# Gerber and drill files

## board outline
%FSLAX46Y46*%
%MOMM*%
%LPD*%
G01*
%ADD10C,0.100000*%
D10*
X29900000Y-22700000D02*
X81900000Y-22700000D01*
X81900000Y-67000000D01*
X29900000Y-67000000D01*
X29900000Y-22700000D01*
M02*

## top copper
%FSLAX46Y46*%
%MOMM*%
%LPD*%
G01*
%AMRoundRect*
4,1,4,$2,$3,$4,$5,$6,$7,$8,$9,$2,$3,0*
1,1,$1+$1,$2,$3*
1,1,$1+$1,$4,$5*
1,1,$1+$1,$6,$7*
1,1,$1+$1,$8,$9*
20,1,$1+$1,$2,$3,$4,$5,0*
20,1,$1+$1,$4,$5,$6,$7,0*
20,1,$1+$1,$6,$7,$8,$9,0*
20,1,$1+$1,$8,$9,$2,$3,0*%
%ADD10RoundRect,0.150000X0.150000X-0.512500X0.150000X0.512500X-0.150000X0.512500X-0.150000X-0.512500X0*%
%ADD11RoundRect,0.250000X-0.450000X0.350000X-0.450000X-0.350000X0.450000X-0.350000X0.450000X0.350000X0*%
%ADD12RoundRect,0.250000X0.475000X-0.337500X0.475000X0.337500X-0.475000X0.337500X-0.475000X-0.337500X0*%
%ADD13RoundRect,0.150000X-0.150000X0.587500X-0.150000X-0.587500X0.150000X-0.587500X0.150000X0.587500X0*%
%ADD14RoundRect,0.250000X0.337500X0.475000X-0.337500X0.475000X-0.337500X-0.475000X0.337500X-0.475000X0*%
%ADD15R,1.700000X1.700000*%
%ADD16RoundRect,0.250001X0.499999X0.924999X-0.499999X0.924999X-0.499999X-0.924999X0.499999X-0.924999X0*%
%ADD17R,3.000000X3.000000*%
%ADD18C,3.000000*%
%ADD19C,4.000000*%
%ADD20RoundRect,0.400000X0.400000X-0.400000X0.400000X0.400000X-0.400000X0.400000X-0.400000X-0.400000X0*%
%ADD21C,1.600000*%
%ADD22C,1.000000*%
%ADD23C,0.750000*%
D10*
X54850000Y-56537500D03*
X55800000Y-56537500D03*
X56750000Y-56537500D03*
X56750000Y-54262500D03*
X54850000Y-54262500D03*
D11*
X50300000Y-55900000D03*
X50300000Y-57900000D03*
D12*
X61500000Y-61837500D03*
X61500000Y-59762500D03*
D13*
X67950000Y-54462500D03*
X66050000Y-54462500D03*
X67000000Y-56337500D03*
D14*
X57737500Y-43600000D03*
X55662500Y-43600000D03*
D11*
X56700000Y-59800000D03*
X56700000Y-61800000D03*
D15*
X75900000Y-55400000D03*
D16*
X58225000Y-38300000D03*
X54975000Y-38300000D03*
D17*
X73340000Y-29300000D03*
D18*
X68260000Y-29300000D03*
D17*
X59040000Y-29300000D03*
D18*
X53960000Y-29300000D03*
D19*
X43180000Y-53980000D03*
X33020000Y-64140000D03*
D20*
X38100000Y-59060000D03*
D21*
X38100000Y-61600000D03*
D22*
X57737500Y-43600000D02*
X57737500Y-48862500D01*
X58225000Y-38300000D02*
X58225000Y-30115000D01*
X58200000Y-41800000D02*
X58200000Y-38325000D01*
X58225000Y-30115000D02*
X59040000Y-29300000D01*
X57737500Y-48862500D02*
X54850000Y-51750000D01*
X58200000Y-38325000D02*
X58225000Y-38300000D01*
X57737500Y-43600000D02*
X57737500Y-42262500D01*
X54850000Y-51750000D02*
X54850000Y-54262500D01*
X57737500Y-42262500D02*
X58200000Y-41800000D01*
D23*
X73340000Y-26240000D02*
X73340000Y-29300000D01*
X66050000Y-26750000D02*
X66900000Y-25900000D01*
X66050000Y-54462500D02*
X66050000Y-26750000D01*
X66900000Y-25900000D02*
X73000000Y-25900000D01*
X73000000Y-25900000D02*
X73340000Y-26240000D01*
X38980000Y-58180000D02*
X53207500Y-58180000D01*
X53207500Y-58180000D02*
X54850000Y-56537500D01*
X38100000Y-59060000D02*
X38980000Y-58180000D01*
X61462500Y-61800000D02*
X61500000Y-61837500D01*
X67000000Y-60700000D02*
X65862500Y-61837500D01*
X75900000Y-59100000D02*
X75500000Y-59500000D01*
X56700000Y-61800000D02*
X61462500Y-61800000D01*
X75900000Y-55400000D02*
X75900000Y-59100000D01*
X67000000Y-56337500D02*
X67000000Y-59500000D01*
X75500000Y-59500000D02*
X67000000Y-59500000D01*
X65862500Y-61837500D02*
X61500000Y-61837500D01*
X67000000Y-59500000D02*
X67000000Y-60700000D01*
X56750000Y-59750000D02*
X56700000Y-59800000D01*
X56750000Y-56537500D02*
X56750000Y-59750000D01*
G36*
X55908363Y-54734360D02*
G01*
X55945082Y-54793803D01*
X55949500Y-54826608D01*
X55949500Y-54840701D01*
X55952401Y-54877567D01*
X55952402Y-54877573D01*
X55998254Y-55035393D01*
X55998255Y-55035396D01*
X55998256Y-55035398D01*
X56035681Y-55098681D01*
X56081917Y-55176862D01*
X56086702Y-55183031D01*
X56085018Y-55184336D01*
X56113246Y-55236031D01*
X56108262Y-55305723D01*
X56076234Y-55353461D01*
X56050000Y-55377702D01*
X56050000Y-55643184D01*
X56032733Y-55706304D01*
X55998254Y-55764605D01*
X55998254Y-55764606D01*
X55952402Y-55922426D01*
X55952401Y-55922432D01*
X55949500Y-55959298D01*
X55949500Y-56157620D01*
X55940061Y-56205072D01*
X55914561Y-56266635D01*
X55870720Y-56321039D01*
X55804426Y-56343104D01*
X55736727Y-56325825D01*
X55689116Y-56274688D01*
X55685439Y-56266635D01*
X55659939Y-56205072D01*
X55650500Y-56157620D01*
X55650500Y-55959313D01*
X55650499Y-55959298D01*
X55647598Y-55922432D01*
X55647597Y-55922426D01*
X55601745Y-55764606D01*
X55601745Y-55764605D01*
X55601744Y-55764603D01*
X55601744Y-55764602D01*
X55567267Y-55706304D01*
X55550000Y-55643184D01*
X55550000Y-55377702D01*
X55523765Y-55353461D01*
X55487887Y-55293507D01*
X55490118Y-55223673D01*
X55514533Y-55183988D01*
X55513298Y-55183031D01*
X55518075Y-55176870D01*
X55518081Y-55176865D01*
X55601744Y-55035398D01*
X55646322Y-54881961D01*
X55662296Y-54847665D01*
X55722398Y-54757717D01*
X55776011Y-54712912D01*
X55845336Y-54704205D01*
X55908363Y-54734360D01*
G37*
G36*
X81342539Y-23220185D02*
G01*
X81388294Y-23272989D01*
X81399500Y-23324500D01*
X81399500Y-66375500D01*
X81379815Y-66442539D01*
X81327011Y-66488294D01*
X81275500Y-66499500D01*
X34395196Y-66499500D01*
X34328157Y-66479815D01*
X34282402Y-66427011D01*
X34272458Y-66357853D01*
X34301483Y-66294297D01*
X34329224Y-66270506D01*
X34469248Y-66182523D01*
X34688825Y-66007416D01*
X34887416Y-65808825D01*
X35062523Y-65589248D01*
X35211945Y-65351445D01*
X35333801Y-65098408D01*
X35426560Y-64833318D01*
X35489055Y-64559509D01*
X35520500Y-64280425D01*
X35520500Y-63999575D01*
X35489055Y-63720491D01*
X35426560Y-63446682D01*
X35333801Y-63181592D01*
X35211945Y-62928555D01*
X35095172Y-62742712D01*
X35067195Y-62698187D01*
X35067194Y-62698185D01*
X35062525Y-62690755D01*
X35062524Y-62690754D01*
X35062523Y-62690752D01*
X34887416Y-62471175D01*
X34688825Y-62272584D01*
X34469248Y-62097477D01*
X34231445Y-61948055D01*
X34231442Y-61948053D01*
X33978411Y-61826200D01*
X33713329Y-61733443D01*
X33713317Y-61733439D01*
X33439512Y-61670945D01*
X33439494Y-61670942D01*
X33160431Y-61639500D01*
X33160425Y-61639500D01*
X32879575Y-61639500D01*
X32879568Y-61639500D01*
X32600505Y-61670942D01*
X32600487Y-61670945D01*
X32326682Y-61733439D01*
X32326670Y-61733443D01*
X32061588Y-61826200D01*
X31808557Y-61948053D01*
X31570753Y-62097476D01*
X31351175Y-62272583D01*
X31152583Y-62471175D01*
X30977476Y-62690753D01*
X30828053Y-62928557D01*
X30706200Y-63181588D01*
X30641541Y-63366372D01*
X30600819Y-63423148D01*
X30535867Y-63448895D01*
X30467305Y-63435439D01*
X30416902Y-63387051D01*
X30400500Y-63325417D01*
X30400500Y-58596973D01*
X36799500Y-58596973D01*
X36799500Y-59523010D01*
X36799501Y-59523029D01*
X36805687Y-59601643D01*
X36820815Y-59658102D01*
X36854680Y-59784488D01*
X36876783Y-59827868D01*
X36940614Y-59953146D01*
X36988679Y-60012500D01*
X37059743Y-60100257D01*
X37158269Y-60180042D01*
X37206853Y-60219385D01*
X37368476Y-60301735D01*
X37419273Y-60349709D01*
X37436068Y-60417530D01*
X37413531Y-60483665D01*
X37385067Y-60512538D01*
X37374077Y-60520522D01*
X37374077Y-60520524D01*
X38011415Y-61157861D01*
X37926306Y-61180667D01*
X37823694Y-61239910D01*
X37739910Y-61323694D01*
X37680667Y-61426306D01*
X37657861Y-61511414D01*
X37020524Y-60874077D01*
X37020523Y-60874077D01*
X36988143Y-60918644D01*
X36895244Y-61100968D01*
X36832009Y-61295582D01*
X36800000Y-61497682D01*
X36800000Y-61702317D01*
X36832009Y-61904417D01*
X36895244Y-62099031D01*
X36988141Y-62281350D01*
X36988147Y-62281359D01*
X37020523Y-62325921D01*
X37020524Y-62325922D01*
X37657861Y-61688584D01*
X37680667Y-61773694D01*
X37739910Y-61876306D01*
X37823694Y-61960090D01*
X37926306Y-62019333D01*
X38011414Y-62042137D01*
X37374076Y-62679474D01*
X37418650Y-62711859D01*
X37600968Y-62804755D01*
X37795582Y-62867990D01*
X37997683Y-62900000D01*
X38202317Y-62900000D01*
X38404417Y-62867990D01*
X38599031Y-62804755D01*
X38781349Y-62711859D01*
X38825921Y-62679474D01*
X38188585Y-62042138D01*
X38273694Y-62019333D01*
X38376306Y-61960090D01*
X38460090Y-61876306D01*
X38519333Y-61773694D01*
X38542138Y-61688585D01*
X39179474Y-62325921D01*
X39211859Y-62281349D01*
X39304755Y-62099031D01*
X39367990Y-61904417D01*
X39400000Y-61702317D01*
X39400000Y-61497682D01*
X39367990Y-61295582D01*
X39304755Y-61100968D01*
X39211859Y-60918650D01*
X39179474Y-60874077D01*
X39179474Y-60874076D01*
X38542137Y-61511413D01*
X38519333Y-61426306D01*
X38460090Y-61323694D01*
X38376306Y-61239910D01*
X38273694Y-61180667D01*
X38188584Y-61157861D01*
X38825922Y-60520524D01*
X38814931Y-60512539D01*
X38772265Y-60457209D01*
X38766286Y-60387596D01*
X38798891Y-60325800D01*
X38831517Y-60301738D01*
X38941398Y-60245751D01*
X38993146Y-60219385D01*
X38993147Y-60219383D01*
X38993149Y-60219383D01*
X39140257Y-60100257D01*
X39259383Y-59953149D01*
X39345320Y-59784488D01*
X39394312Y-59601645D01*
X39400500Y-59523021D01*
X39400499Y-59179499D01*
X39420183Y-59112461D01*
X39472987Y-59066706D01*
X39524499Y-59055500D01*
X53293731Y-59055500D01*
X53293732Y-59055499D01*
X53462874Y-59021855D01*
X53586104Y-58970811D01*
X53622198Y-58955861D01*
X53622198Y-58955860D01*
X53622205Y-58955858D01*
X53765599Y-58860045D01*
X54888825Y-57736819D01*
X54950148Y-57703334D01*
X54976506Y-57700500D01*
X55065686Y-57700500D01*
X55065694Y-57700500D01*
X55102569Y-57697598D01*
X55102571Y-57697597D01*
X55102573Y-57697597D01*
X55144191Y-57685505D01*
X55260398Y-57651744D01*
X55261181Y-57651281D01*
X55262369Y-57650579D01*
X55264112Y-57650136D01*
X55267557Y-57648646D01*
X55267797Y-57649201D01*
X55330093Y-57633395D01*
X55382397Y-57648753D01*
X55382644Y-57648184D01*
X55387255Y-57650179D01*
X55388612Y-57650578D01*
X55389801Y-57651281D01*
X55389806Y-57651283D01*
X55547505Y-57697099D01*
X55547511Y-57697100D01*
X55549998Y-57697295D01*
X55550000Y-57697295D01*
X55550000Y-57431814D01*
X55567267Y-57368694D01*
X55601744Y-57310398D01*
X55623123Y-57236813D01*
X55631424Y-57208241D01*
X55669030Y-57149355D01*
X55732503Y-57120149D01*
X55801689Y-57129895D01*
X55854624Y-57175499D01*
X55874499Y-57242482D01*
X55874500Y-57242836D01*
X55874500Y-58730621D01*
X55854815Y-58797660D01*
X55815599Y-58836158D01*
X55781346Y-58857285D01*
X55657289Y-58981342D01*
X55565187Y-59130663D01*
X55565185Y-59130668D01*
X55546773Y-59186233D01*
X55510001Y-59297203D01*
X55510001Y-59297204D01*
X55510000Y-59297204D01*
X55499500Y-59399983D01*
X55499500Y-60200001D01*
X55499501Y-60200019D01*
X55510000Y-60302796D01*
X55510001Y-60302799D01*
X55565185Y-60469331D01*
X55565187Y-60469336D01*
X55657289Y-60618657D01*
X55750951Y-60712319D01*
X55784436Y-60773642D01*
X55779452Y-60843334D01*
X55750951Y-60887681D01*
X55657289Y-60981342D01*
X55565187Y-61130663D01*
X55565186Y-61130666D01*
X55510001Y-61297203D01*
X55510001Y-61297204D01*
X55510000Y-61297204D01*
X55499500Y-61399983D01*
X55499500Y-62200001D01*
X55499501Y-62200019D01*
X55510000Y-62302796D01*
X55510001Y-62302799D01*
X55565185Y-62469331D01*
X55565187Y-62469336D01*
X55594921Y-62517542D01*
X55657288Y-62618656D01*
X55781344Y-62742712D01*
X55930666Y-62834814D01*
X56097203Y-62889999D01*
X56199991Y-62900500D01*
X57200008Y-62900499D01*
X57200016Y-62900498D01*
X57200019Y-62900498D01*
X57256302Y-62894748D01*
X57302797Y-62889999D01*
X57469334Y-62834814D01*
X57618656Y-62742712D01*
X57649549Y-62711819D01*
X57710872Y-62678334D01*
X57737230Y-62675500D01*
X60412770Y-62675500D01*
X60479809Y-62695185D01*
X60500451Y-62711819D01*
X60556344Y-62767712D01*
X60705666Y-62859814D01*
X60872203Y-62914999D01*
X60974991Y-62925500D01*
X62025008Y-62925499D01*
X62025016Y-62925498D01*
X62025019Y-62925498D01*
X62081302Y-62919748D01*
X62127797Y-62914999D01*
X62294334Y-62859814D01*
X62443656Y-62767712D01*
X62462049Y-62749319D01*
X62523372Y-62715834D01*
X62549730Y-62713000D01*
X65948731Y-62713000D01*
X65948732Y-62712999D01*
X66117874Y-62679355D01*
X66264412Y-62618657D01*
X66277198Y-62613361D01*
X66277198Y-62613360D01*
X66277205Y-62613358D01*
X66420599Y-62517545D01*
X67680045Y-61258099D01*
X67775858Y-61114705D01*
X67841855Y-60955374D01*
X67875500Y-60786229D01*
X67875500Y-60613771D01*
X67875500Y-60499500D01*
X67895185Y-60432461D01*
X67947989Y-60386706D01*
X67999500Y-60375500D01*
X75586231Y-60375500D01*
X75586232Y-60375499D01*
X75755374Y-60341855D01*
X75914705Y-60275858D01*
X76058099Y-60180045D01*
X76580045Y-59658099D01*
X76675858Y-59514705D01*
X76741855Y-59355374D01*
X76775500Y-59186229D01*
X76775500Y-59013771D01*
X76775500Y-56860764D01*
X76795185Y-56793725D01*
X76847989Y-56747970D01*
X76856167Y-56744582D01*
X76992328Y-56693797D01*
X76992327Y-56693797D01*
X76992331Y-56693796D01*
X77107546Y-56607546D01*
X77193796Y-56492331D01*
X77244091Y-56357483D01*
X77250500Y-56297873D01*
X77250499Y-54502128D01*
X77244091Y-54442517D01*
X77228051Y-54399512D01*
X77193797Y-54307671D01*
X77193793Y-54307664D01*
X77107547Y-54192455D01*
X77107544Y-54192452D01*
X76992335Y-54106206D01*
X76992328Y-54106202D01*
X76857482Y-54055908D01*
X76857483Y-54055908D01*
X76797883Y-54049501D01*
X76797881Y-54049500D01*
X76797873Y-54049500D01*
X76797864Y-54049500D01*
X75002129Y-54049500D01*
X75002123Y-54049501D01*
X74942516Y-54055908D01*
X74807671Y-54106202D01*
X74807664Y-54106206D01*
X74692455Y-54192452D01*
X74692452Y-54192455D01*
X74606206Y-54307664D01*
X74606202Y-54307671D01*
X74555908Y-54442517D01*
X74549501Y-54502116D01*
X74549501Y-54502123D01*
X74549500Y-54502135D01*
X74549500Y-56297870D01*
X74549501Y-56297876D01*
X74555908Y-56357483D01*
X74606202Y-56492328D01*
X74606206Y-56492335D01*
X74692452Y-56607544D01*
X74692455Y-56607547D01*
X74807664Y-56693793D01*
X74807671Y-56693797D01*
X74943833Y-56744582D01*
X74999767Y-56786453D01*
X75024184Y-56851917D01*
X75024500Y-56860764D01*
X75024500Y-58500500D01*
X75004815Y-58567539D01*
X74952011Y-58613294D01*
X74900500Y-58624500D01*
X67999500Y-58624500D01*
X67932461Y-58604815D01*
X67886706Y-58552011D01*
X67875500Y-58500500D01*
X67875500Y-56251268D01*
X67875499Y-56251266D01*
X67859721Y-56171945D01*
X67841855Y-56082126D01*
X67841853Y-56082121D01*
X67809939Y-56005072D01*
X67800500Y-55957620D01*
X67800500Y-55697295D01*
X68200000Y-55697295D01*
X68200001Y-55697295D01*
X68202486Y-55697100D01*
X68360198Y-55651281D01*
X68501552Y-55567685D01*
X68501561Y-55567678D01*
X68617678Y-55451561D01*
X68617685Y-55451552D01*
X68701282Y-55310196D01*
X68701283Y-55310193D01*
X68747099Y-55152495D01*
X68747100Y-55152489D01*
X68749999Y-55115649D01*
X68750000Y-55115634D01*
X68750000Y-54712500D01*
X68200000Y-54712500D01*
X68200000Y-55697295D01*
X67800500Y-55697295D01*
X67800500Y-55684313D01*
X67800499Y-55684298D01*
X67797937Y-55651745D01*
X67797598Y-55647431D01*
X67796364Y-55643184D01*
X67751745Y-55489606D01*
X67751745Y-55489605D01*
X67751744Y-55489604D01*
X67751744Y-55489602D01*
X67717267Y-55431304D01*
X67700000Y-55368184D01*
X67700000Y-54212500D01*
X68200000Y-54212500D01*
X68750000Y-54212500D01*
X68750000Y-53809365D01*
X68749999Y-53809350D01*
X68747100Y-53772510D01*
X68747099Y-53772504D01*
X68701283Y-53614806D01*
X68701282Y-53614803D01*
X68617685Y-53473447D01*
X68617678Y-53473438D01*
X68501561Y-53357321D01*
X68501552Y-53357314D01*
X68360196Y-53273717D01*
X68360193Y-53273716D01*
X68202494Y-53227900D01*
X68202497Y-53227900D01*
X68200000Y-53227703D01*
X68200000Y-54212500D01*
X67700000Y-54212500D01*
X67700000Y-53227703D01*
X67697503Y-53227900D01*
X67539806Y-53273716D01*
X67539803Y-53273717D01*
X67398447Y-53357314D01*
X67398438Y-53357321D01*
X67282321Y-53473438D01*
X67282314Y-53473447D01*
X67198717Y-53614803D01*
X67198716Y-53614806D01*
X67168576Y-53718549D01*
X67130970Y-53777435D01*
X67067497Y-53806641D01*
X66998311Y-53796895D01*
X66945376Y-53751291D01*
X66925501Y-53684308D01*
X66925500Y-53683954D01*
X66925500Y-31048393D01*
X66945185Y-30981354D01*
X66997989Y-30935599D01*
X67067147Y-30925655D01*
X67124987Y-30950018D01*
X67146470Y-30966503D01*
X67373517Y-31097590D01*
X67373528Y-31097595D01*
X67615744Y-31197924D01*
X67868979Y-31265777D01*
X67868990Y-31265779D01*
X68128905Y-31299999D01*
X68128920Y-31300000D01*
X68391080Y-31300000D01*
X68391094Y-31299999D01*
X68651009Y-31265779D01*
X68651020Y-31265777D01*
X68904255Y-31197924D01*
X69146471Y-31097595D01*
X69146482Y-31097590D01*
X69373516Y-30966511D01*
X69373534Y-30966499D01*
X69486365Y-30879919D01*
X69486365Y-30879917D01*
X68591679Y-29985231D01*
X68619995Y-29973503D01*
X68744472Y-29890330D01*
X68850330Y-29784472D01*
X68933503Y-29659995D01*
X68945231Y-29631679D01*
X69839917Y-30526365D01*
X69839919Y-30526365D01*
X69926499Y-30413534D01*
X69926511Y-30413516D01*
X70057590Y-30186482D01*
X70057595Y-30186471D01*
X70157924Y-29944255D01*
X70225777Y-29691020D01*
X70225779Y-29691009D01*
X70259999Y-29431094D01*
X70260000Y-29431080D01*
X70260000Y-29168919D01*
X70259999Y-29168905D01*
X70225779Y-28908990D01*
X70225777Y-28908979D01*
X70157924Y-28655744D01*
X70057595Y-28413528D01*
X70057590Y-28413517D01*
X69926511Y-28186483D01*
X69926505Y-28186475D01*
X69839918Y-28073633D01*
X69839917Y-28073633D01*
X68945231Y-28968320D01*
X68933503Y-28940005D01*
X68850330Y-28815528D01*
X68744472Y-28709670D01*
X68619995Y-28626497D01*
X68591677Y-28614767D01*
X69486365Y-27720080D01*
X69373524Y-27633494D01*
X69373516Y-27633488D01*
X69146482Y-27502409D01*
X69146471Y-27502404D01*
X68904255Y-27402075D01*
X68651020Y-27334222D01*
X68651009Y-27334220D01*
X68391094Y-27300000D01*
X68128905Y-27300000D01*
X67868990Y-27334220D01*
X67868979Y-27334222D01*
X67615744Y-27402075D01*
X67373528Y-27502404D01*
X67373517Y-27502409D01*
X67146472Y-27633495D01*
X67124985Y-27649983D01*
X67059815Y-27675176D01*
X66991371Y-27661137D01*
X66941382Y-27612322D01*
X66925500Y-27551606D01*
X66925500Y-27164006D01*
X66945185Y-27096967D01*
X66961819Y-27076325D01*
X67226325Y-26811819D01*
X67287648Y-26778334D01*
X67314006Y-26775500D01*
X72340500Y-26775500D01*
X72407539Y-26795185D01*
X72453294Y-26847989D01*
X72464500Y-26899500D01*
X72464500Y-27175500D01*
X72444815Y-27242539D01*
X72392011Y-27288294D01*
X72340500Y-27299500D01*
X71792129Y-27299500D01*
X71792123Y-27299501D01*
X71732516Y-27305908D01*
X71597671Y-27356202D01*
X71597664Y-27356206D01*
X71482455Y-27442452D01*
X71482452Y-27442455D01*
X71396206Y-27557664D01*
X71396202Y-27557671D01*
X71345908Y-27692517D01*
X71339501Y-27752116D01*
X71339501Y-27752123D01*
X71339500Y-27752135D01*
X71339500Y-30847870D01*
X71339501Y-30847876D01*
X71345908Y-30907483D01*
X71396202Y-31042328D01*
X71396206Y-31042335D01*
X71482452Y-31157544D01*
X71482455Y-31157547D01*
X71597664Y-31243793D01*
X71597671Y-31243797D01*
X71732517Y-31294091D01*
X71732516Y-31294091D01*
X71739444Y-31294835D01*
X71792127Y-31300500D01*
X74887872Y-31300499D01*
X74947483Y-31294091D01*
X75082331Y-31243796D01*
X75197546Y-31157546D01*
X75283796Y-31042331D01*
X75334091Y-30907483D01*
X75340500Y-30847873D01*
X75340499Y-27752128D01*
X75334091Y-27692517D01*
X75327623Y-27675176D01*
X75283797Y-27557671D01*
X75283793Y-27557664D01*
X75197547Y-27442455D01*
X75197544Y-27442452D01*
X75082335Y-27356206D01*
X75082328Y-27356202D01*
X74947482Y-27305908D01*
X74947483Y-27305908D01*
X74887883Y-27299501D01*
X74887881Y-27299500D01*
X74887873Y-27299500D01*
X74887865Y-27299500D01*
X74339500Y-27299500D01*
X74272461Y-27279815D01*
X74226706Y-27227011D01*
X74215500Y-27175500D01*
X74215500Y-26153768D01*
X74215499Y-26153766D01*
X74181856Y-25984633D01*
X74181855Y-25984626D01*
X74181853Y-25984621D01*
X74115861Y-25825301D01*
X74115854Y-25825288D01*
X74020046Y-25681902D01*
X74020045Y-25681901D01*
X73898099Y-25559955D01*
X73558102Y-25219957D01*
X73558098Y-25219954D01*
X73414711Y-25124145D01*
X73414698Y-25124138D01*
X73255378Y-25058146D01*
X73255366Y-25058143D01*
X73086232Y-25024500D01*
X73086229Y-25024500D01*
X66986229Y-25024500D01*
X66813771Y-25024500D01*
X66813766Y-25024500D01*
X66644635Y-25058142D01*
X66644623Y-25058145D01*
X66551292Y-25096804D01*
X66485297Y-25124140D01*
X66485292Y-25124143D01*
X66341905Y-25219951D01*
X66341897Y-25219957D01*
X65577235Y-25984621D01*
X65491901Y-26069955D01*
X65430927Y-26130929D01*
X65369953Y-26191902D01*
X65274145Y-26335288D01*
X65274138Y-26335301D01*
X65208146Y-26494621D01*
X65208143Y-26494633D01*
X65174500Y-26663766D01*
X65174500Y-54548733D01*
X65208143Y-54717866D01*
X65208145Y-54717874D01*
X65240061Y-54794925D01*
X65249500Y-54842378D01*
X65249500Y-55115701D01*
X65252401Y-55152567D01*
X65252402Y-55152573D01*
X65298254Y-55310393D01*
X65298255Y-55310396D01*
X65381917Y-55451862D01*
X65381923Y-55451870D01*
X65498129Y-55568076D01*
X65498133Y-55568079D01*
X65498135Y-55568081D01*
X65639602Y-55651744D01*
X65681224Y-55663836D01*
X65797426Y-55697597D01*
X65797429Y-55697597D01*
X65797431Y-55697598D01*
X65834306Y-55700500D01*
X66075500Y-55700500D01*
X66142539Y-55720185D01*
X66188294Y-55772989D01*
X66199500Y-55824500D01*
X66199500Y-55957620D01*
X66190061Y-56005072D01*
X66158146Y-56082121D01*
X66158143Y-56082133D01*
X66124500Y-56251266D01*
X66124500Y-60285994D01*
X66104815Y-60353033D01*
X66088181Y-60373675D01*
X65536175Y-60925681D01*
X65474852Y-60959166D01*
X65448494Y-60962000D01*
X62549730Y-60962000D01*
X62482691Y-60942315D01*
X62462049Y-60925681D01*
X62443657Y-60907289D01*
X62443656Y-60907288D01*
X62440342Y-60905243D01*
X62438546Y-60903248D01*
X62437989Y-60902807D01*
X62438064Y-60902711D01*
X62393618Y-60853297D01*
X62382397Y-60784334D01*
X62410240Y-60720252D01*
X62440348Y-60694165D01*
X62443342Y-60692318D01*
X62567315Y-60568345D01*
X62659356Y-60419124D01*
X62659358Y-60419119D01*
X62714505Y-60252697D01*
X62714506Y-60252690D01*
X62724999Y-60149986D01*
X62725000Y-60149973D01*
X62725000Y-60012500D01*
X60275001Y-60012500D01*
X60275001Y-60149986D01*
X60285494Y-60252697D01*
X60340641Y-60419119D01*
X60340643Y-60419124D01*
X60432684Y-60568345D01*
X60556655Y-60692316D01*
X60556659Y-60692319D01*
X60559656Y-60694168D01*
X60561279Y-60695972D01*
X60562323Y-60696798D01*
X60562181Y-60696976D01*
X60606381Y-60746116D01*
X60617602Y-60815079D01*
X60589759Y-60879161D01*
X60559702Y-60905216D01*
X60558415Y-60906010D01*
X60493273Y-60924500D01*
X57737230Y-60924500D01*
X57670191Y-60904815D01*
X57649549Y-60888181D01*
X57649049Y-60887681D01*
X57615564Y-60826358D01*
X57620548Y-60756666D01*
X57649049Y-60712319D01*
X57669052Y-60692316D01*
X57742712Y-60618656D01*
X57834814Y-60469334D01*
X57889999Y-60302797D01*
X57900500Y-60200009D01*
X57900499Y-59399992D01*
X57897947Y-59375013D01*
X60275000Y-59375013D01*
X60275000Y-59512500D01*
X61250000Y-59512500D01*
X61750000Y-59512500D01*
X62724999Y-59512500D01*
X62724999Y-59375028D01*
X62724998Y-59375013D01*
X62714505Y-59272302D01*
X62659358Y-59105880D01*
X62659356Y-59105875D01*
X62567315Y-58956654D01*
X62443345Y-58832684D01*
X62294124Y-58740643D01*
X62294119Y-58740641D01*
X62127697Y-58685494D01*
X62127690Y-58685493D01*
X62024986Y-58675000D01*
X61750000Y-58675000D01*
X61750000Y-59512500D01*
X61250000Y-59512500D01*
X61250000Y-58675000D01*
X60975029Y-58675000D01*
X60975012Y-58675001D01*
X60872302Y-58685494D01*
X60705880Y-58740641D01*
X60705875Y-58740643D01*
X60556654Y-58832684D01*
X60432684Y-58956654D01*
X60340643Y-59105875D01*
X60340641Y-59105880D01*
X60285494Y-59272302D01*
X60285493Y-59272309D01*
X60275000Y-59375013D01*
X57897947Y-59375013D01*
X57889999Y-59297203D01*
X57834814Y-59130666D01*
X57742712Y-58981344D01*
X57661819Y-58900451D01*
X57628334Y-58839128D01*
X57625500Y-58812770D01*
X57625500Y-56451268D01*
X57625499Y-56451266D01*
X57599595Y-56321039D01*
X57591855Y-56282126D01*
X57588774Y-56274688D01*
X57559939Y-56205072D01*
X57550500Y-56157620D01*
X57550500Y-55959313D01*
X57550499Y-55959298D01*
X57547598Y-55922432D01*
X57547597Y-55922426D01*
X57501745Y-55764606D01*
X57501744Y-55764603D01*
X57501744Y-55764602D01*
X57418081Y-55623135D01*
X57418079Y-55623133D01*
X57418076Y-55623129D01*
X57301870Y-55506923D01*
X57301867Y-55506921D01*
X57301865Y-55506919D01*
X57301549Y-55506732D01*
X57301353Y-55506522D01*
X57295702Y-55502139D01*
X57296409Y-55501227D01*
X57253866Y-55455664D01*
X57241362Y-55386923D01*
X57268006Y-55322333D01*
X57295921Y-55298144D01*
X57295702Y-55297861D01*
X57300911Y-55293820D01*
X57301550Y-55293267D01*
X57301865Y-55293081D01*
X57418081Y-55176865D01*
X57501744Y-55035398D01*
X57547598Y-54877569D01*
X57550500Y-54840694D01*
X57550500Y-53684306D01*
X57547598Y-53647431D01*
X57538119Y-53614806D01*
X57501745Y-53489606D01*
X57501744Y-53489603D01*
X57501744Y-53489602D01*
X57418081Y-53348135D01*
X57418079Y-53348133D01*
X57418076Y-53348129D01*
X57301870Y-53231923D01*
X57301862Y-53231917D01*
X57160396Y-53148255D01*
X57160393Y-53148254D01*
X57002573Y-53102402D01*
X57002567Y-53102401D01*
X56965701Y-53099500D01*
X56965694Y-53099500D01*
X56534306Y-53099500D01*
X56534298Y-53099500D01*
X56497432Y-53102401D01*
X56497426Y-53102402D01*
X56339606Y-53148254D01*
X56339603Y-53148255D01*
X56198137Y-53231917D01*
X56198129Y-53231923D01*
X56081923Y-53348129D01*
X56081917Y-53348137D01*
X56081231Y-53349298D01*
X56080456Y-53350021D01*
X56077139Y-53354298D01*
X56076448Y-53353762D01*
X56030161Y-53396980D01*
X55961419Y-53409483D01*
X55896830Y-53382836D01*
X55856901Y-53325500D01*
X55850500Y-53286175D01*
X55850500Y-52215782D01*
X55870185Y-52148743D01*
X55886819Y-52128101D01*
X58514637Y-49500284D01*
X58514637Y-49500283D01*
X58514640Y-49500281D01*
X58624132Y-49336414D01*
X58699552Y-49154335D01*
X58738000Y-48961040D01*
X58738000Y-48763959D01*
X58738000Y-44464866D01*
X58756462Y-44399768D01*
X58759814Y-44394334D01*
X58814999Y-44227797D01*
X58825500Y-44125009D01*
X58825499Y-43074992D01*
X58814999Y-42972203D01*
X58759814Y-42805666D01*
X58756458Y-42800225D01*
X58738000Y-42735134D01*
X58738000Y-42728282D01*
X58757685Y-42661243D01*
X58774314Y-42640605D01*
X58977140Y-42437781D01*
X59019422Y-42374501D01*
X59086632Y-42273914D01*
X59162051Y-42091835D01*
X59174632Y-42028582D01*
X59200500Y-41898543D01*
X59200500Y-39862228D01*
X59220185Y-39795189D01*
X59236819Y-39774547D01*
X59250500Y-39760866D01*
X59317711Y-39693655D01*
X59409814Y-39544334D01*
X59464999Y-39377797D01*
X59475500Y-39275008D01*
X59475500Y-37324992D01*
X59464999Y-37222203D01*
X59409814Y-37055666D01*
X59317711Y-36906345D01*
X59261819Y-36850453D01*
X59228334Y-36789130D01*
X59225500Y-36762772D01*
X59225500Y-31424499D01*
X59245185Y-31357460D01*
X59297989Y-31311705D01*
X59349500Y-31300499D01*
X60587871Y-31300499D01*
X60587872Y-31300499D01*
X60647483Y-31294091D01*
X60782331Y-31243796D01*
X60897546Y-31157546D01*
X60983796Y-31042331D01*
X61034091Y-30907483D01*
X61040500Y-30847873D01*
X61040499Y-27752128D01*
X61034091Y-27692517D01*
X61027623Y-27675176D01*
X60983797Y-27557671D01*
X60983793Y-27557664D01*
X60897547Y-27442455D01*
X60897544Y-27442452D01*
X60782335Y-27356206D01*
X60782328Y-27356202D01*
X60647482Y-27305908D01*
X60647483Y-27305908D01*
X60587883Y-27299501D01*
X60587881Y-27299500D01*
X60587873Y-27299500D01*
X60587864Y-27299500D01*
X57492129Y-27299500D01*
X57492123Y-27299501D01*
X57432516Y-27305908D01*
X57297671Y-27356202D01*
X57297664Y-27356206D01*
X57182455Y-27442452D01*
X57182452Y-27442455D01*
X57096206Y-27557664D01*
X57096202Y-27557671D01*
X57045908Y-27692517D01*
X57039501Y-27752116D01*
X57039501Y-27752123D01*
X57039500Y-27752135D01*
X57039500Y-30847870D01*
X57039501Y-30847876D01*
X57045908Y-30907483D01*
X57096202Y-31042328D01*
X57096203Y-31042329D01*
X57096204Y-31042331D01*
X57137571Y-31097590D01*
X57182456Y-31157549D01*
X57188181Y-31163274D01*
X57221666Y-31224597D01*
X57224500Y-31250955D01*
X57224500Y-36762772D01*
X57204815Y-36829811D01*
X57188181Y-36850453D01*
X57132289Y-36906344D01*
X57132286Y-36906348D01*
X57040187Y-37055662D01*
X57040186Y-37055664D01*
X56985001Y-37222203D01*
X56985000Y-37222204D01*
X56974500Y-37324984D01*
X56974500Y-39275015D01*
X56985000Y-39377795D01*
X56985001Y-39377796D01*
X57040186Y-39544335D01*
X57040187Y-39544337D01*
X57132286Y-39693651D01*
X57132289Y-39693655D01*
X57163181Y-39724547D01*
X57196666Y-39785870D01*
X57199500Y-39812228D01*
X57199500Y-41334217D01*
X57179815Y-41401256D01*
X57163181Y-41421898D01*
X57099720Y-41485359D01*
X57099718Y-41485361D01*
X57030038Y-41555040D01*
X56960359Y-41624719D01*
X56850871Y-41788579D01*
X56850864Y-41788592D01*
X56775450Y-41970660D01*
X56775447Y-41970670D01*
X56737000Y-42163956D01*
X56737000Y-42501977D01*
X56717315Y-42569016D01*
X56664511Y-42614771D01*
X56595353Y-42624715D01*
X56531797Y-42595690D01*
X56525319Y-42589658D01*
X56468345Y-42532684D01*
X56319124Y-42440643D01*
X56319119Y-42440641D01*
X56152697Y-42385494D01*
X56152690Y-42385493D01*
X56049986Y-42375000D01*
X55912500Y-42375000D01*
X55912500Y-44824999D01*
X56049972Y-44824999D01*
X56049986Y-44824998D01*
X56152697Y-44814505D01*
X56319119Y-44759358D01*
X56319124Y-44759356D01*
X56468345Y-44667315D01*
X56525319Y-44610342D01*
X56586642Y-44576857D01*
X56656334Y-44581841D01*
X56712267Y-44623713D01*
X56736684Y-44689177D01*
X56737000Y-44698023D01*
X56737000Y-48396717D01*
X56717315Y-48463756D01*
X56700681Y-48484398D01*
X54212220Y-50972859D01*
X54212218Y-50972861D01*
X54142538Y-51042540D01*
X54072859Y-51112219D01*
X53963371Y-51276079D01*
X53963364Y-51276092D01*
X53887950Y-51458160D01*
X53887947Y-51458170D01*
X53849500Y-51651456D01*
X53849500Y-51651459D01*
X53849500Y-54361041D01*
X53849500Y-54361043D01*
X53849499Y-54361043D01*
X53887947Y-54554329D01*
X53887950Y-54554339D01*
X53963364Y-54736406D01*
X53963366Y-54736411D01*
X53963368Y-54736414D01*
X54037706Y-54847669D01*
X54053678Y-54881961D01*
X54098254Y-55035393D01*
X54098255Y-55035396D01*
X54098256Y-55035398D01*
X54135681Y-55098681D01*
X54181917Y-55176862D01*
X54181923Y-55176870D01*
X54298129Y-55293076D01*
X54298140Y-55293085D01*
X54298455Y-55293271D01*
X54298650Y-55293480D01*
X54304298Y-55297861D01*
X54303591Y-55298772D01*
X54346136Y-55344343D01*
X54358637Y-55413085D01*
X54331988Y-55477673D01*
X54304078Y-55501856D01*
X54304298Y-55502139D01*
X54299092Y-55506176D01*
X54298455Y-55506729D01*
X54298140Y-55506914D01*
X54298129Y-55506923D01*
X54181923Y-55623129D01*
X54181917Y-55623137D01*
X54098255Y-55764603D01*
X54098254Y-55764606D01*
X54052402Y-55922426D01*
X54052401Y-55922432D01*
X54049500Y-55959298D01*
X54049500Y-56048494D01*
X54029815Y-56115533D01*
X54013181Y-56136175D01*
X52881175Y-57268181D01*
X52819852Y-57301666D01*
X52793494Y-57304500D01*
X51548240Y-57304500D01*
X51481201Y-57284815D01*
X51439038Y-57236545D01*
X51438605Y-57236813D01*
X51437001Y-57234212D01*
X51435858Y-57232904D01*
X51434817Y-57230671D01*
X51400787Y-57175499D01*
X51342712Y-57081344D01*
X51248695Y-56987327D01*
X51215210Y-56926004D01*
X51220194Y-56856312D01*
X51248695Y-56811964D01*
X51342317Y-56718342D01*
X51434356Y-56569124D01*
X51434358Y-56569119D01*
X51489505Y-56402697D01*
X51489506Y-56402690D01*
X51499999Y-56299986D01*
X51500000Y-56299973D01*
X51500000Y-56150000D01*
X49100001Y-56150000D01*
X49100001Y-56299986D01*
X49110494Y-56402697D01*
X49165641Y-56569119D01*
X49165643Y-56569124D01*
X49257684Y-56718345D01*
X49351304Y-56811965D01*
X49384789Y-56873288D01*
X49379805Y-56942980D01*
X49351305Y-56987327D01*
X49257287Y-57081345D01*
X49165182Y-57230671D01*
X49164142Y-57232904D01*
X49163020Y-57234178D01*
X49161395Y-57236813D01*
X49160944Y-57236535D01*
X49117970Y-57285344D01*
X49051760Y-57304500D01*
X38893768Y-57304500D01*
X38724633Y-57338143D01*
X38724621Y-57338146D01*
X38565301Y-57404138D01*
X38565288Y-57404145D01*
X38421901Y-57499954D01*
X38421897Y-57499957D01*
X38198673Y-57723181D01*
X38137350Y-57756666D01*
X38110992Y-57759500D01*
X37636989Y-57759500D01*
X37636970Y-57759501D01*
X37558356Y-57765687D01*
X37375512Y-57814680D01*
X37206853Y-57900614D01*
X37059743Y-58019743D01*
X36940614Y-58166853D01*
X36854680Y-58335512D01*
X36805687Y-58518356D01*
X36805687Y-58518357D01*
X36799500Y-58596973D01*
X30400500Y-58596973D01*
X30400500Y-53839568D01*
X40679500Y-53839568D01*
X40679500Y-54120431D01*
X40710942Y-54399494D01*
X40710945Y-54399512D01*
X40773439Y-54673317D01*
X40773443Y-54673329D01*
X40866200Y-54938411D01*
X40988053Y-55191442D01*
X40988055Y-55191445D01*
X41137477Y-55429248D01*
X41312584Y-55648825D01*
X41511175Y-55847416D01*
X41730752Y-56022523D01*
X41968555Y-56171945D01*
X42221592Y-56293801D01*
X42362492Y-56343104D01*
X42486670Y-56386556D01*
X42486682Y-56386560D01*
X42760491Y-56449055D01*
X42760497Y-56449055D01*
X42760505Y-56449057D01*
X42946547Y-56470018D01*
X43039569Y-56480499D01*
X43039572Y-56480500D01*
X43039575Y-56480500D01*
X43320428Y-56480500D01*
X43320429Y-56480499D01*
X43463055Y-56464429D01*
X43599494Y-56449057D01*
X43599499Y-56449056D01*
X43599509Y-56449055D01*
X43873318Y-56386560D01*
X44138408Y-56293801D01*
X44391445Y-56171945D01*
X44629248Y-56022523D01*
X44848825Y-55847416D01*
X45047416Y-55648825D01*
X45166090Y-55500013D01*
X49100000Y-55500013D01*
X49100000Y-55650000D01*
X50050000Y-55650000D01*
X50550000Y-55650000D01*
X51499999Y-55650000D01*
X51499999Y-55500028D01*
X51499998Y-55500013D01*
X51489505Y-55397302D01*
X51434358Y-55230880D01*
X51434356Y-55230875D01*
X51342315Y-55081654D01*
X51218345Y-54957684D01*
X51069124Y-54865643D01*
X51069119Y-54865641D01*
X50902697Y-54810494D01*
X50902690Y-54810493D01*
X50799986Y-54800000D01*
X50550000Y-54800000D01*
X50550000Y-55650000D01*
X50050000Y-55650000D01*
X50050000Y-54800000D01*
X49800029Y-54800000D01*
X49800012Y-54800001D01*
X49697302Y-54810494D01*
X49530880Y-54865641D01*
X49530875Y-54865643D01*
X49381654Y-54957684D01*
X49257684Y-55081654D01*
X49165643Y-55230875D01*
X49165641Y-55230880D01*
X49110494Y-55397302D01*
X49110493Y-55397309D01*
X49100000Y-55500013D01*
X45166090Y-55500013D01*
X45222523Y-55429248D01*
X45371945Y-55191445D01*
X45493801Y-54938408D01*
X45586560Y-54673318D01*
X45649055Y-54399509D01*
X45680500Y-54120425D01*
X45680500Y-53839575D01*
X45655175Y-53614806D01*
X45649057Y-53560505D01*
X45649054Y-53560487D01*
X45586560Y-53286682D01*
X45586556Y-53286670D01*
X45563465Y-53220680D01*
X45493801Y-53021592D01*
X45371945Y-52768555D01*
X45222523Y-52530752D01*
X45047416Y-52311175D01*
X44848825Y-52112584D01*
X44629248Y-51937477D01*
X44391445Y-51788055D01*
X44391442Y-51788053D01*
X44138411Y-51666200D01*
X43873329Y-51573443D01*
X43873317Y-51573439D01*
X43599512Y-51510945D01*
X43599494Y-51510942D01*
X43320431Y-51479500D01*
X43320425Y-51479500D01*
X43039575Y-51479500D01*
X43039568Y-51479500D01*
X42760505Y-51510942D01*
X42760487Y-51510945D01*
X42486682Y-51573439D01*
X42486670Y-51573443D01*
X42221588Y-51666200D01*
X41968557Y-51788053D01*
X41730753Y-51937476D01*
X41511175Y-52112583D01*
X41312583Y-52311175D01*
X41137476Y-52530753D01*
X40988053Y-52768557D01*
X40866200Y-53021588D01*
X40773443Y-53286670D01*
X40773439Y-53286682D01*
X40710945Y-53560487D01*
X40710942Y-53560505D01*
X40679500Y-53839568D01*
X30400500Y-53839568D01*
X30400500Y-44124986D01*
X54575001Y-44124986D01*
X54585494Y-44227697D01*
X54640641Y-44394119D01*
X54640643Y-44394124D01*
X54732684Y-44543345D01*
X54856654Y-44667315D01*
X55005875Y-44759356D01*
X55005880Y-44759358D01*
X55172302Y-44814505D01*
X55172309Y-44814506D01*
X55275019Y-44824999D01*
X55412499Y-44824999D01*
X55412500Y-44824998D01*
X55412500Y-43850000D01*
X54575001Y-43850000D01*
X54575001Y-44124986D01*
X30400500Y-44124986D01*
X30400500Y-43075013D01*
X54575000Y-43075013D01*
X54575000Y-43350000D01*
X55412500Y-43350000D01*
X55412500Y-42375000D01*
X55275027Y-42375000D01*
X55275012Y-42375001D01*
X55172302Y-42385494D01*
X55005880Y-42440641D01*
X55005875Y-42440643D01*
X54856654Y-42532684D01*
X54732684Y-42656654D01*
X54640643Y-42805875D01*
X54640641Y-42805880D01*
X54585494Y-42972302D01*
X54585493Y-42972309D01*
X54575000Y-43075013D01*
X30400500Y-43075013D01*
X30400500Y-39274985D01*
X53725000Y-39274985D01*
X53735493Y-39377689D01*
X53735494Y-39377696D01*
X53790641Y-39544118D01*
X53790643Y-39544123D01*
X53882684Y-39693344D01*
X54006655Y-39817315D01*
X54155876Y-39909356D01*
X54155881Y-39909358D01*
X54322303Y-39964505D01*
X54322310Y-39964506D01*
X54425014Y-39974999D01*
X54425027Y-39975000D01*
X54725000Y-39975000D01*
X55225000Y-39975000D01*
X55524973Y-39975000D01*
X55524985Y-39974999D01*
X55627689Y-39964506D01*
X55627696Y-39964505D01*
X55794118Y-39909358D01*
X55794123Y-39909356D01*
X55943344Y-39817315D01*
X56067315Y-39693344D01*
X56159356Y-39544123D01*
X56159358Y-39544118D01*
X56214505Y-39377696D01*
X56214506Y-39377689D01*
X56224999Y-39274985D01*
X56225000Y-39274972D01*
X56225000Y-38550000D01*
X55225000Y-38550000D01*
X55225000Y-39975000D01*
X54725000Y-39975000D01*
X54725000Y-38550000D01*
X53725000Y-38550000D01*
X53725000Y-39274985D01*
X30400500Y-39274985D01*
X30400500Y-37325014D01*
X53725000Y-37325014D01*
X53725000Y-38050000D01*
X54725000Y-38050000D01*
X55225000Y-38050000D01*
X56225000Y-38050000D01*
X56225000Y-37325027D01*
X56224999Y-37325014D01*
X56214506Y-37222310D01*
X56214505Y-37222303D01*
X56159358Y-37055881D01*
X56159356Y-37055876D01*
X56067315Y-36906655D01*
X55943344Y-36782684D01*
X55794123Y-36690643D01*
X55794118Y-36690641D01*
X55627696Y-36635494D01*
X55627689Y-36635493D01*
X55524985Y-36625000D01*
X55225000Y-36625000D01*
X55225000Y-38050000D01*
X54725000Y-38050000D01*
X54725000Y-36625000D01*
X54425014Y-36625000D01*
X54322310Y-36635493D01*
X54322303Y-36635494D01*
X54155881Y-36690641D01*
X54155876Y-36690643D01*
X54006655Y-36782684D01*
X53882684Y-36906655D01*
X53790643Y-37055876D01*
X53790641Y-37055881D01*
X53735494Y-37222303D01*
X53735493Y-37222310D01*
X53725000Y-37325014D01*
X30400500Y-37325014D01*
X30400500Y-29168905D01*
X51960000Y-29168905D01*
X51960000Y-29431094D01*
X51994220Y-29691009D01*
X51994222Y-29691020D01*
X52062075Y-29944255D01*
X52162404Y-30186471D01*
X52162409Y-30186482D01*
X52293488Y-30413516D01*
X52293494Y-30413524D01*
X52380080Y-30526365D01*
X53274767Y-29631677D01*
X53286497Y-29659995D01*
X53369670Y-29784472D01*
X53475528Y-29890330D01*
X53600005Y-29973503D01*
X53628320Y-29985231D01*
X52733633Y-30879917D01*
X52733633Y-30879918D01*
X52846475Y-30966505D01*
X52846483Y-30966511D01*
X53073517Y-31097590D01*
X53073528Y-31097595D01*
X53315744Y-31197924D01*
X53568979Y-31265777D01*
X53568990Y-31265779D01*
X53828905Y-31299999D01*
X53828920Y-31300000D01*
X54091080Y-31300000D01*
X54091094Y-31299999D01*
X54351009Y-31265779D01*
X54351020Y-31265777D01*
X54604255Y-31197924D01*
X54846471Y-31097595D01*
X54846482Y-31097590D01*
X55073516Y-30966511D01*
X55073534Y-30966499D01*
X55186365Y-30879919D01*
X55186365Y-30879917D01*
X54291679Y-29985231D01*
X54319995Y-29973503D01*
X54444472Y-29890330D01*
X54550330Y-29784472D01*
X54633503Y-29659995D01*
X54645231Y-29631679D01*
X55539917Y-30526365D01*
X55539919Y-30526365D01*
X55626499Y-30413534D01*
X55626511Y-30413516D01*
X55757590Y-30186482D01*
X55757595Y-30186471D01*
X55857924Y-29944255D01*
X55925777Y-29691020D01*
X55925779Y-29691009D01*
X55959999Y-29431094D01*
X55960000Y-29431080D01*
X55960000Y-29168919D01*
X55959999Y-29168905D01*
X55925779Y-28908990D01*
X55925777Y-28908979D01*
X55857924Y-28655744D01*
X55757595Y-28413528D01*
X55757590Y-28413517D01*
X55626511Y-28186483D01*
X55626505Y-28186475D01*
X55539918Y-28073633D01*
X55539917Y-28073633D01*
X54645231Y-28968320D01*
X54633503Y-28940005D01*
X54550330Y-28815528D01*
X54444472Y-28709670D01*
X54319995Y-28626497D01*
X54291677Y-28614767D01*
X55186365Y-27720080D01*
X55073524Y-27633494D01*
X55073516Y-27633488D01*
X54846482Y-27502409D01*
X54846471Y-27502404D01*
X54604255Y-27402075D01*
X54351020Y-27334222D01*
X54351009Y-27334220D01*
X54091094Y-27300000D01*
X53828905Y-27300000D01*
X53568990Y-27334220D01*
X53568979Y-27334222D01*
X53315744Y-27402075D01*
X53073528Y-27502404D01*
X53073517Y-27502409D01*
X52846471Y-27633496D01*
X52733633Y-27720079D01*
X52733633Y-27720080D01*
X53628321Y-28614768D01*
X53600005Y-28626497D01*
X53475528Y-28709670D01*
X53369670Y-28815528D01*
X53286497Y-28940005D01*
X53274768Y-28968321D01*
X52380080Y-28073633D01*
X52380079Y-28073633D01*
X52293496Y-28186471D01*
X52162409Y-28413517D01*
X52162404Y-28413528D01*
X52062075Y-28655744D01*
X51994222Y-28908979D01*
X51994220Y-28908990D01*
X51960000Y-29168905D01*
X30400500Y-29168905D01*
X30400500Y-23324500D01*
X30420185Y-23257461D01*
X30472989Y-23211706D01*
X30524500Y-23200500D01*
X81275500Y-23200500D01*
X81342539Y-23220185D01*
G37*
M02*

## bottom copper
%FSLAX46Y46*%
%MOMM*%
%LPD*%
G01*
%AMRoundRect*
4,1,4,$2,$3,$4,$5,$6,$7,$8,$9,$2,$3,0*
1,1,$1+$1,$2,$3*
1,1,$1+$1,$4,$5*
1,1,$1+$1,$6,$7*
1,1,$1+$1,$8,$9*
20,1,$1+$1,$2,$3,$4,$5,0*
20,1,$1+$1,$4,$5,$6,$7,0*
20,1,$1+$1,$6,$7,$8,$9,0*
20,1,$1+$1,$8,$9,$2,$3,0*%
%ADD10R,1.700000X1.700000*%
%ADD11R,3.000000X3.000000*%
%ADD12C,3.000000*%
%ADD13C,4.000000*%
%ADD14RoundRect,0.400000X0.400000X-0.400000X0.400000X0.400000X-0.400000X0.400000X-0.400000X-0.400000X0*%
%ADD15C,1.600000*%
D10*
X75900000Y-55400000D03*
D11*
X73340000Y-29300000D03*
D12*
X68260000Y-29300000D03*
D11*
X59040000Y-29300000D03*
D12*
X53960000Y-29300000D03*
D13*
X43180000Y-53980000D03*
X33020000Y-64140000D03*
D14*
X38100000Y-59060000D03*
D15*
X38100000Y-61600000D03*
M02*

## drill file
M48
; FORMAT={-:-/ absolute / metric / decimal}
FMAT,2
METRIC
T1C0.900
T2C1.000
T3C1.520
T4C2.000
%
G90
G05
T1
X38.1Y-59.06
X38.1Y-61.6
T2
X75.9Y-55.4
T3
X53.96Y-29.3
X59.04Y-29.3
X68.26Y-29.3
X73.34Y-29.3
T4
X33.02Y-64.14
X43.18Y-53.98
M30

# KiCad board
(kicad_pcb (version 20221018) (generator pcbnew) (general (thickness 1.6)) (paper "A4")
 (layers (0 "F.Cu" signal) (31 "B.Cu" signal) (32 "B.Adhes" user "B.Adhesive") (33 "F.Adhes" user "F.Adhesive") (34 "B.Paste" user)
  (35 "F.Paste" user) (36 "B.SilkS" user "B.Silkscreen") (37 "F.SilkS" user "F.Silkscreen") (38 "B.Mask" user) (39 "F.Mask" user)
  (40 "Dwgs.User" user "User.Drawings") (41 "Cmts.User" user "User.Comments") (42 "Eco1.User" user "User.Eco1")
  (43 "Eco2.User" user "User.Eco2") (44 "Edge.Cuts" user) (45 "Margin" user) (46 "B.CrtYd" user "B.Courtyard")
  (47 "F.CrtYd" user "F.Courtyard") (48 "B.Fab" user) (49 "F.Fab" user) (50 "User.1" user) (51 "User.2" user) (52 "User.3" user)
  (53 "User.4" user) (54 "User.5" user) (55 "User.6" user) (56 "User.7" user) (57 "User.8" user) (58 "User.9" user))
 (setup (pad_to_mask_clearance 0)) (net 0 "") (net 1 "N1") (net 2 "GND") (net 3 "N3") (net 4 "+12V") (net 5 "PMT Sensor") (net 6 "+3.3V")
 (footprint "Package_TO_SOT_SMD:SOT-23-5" (layer "F.Cu") (at 55.8 55.4 90)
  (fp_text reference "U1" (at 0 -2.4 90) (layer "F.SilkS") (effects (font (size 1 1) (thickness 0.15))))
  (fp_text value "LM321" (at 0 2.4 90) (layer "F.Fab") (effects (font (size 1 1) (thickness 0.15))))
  (pad "1" smd roundrect (at -1.1375 -0.95 90) (size 1.325 0.6) (layers "F.Cu" "F.Paste" "F.Mask") (roundrect_rratio 0.25) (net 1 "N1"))
  (pad "2" smd roundrect (at -1.1375 0 90) (size 1.325 0.6) (layers "F.Cu" "F.Paste" "F.Mask") (roundrect_rratio 0.25) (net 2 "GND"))
  (pad "3" smd roundrect (at -1.1375 0.95 90) (size 1.325 0.6) (layers "F.Cu" "F.Paste" "F.Mask") (roundrect_rratio 0.25) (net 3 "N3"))
  (pad "4" smd roundrect (at 1.1375 0.95 90) (size 1.325 0.6) (layers "F.Cu" "F.Paste" "F.Mask") (roundrect_rratio 0.25) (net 3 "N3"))
  (pad "5" smd roundrect (at 1.1375 -0.95 90) (size 1.325 0.6) (layers "F.Cu" "F.Paste" "F.Mask") (roundrect_rratio 0.25) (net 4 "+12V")))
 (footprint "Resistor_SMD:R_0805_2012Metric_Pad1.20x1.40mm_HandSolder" (layer "F.Cu") (at 50.3 56.9 -90)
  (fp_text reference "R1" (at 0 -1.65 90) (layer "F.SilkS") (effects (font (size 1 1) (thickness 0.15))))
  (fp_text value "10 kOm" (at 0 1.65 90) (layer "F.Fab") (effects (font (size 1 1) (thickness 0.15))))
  (pad "1" smd roundrect (at -1 0 270) (size 1.2 1.4) (layers "F.Cu" "F.Paste" "F.Mask") (roundrect_rratio 0.208333) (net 2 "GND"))
  (pad "2" smd roundrect (at 1 0 270) (size 1.2 1.4) (layers "F.Cu" "F.Paste" "F.Mask") (roundrect_rratio 0.208333) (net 1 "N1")))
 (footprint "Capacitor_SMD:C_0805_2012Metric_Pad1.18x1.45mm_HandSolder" (layer "F.Cu") (at 61.5 60.8 90)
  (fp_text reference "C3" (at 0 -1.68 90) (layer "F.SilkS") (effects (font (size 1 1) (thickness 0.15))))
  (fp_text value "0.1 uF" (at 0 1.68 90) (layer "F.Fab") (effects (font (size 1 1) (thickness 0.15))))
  (pad "1" smd roundrect (at -1.0375 0 90) (size 1.175 1.45) (layers "F.Cu" "F.Paste" "F.Mask") (roundrect_rratio 0.212766)
   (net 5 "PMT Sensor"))
  (pad "2" smd roundrect (at 1.0375 0 90) (size 1.175 1.45) (layers "F.Cu" "F.Paste" "F.Mask") (roundrect_rratio 0.212766) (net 2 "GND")))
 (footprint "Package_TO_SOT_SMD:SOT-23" (layer "F.Cu") (at 67 55.4 -90)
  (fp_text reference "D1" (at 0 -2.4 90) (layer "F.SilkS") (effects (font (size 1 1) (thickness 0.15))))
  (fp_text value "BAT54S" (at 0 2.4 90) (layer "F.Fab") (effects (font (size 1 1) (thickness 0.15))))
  (pad "1" smd roundrect (at -0.9375 -0.95 270) (size 1.475 0.6) (layers "F.Cu" "F.Paste" "F.Mask") (roundrect_rratio 0.25) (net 2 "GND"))
  (pad "2" smd roundrect (at -0.9375 0.95 270) (size 1.475 0.6) (layers "F.Cu" "F.Paste" "F.Mask") (roundrect_rratio 0.25) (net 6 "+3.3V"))
  (pad "3" smd roundrect (at 0.9375 0 270) (size 1.475 0.6) (layers "F.Cu" "F.Paste" "F.Mask") (roundrect_rratio 0.25) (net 5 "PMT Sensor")))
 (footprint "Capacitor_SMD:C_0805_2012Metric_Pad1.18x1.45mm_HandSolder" (layer "F.Cu") (at 56.7 43.6 180)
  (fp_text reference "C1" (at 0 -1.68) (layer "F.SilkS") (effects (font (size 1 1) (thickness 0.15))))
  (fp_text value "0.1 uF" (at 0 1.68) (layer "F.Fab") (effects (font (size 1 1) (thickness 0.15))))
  (pad "1" smd roundrect (at -1.0375 0 180) (size 1.175 1.45) (layers "F.Cu" "F.Paste" "F.Mask") (roundrect_rratio 0.212766) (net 4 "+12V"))
  (pad "2" smd roundrect (at 1.0375 0 180) (size 1.175 1.45) (layers "F.Cu" "F.Paste" "F.Mask") (roundrect_rratio 0.212766) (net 2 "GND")))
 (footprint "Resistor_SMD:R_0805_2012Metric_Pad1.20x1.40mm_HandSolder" (layer "F.Cu") (at 56.7 60.8 -90)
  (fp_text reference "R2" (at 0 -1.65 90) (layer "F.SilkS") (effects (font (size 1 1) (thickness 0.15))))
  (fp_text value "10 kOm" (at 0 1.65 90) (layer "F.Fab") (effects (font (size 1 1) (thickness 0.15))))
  (pad "1" smd roundrect (at -1 0 270) (size 1.2 1.4) (layers "F.Cu" "F.Paste" "F.Mask") (roundrect_rratio 0.208333) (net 3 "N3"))
  (pad "2" smd roundrect (at 1 0 270) (size 1.2 1.4) (layers "F.Cu" "F.Paste" "F.Mask") (roundrect_rratio 0.208333) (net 5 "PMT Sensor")))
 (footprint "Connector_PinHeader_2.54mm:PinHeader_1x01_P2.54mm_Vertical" (layer "F.Cu") (at 75.9 55.4)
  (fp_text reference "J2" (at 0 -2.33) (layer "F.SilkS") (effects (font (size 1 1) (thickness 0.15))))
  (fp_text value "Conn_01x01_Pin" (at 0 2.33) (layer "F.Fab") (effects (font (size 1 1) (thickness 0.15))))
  (pad "1" thru_hole rect (at 0 0) (size 1.7 1.7) (drill 1) (layers "*.Cu" "*.Mask") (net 5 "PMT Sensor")))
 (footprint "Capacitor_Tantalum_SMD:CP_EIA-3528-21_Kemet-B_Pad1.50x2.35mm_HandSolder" (layer "F.Cu") (at 56.6 38.3 180)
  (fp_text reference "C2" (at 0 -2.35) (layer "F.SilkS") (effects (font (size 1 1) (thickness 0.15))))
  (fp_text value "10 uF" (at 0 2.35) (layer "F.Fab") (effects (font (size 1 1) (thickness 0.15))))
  (pad "1" smd roundrect (at -1.625 0 180) (size 1.5 2.35) (layers "F.Cu" "F.Paste" "F.Mask") (roundrect_rratio 0.166667) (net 4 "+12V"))
  (pad "2" smd roundrect (at 1.625 0 180) (size 1.5 2.35) (layers "F.Cu" "F.Paste" "F.Mask") (roundrect_rratio 0.166667) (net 2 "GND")))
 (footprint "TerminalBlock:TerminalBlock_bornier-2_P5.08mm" (layer "B.Cu") (at 73.34 29.3 180)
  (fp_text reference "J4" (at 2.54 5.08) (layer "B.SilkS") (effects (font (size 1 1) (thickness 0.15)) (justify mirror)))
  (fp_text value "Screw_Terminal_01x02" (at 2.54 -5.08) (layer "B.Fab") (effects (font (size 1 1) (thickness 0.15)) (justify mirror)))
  (pad "1" thru_hole rect (at 0 0 180) (size 3 3) (drill 1.52) (layers "*.Cu" "*.Mask") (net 6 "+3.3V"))
  (pad "2" thru_hole circle (at 5.08 0 180) (size 3 3) (drill 1.52) (layers "*.Cu" "*.Mask") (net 2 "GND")))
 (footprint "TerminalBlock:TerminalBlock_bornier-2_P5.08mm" (layer "B.Cu") (at 59.04 29.3 180)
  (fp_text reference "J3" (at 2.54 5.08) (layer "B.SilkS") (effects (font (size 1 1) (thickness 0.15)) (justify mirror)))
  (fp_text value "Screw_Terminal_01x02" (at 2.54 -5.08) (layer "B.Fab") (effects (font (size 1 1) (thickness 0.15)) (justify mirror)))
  (pad "1" thru_hole rect (at 0 0 180) (size 3 3) (drill 1.52) (layers "*.Cu" "*.Mask") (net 4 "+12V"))
  (pad "2" thru_hole circle (at 5.08 0 180) (size 3 3) (drill 1.52) (layers "*.Cu" "*.Mask") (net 2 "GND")))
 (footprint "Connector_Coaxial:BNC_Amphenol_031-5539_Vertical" (layer "B.Cu") (at 38.1 59.06 -90)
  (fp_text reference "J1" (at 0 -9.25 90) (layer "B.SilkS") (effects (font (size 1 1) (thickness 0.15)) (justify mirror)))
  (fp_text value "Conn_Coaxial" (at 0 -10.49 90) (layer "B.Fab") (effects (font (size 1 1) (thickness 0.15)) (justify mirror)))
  (pad "" thru_hole circle (at -5.08 -5.08 90) (size 4 4) (drill 2) (layers "*.Cu" "*.Mask"))
  (pad "" thru_hole circle (at 5.08 5.08 90) (size 4 4) (drill 2) (layers "*.Cu" "*.Mask"))
  (pad "1" thru_hole roundrect (at 0 0 90) (size 1.6 1.6) (drill 0.9) (layers "*.Cu" "*.Mask") (roundrect_rratio 0.25) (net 1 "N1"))
  (pad "2" thru_hole circle (at 2.54 0 90) (size 1.6 1.6) (drill 0.9) (layers "*.Cu" "*.Mask") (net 2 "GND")))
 (gr_rect (start 29.9 22.7) (end 81.9 67) (stroke (width 0.1) (type default)) (fill none) (layer "Edge.Cuts"))
 (segment (start 57.7375 43.6) (end 57.7375 48.8625) (width 1) (layer "F.Cu") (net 4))
 (segment (start 58.225 38.3) (end 58.225 30.115) (width 1) (layer "F.Cu") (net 4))
 (segment (start 58.2 41.8) (end 58.2 38.325) (width 1) (layer "F.Cu") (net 4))
 (segment (start 58.225 30.115) (end 59.04 29.3) (width 1) (layer "F.Cu") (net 4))
 (segment (start 57.7375 48.8625) (end 54.85 51.75) (width 1) (layer "F.Cu") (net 4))
 (segment (start 58.2 38.325) (end 58.225 38.3) (width 1) (layer "F.Cu") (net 4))
 (segment (start 57.7375 43.6) (end 57.7375 42.2625) (width 1) (layer "F.Cu") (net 4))
 (segment (start 54.85 51.75) (end 54.85 54.2625) (width 1) (layer "F.Cu") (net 4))
 (segment (start 57.7375 42.2625) (end 58.2 41.8) (width 1) (layer "F.Cu") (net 4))
 (segment (start 73.34 26.24) (end 73.34 29.3) (width 0.75) (layer "F.Cu") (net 6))
 (segment (start 66.05 26.75) (end 66.9 25.9) (width 0.75) (layer "F.Cu") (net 6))
 (segment (start 66.05 54.4625) (end 66.05 26.75) (width 0.75) (layer "F.Cu") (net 6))
 (segment (start 66.9 25.9) (end 73 25.9) (width 0.75) (layer "F.Cu") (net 6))
 (segment (start 73 25.9) (end 73.34 26.24) (width 0.75) (layer "F.Cu") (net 6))
 (segment (start 38.98 58.18) (end 53.2075 58.18) (width 0.75) (layer "F.Cu") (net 1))
 (segment (start 53.2075 58.18) (end 54.85 56.5375) (width 0.75) (layer "F.Cu") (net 1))
 (segment (start 38.1 59.06) (end 38.98 58.18) (width 0.75) (layer "F.Cu") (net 1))
 (segment (start 61.4625 61.8) (end 61.5 61.8375) (width 0.75) (layer "F.Cu") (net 5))
 (segment (start 67 60.7) (end 65.8625 61.8375) (width 0.75) (layer "F.Cu") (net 5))
 (segment (start 75.9 59.1) (end 75.5 59.5) (width 0.75) (layer "F.Cu") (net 5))
 (segment (start 56.7 61.8) (end 61.4625 61.8) (width 0.75) (layer "F.Cu") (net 5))
 (segment (start 75.9 55.4) (end 75.9 59.1) (width 0.75) (layer "F.Cu") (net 5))
 (segment (start 67 56.3375) (end 67 59.5) (width 0.75) (layer "F.Cu") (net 5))
 (segment (start 75.5 59.5) (end 67 59.5) (width 0.75) (layer "F.Cu") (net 5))
 (segment (start 65.8625 61.8375) (end 61.5 61.8375) (width 0.75) (layer "F.Cu") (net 5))
 (segment (start 67 59.5) (end 67 60.7) (width 0.75) (layer "F.Cu") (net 5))
 (segment (start 56.75 59.75) (end 56.7 59.8) (width 0.75) (layer "F.Cu") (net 3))
 (segment (start 56.75 56.5375) (end 56.75 59.75) (width 0.75) (layer "F.Cu") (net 3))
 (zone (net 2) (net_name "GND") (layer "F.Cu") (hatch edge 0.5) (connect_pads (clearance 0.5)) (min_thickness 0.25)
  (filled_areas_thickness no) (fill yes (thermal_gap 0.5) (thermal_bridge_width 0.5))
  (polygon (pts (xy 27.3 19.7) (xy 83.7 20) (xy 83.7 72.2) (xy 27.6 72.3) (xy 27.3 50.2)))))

